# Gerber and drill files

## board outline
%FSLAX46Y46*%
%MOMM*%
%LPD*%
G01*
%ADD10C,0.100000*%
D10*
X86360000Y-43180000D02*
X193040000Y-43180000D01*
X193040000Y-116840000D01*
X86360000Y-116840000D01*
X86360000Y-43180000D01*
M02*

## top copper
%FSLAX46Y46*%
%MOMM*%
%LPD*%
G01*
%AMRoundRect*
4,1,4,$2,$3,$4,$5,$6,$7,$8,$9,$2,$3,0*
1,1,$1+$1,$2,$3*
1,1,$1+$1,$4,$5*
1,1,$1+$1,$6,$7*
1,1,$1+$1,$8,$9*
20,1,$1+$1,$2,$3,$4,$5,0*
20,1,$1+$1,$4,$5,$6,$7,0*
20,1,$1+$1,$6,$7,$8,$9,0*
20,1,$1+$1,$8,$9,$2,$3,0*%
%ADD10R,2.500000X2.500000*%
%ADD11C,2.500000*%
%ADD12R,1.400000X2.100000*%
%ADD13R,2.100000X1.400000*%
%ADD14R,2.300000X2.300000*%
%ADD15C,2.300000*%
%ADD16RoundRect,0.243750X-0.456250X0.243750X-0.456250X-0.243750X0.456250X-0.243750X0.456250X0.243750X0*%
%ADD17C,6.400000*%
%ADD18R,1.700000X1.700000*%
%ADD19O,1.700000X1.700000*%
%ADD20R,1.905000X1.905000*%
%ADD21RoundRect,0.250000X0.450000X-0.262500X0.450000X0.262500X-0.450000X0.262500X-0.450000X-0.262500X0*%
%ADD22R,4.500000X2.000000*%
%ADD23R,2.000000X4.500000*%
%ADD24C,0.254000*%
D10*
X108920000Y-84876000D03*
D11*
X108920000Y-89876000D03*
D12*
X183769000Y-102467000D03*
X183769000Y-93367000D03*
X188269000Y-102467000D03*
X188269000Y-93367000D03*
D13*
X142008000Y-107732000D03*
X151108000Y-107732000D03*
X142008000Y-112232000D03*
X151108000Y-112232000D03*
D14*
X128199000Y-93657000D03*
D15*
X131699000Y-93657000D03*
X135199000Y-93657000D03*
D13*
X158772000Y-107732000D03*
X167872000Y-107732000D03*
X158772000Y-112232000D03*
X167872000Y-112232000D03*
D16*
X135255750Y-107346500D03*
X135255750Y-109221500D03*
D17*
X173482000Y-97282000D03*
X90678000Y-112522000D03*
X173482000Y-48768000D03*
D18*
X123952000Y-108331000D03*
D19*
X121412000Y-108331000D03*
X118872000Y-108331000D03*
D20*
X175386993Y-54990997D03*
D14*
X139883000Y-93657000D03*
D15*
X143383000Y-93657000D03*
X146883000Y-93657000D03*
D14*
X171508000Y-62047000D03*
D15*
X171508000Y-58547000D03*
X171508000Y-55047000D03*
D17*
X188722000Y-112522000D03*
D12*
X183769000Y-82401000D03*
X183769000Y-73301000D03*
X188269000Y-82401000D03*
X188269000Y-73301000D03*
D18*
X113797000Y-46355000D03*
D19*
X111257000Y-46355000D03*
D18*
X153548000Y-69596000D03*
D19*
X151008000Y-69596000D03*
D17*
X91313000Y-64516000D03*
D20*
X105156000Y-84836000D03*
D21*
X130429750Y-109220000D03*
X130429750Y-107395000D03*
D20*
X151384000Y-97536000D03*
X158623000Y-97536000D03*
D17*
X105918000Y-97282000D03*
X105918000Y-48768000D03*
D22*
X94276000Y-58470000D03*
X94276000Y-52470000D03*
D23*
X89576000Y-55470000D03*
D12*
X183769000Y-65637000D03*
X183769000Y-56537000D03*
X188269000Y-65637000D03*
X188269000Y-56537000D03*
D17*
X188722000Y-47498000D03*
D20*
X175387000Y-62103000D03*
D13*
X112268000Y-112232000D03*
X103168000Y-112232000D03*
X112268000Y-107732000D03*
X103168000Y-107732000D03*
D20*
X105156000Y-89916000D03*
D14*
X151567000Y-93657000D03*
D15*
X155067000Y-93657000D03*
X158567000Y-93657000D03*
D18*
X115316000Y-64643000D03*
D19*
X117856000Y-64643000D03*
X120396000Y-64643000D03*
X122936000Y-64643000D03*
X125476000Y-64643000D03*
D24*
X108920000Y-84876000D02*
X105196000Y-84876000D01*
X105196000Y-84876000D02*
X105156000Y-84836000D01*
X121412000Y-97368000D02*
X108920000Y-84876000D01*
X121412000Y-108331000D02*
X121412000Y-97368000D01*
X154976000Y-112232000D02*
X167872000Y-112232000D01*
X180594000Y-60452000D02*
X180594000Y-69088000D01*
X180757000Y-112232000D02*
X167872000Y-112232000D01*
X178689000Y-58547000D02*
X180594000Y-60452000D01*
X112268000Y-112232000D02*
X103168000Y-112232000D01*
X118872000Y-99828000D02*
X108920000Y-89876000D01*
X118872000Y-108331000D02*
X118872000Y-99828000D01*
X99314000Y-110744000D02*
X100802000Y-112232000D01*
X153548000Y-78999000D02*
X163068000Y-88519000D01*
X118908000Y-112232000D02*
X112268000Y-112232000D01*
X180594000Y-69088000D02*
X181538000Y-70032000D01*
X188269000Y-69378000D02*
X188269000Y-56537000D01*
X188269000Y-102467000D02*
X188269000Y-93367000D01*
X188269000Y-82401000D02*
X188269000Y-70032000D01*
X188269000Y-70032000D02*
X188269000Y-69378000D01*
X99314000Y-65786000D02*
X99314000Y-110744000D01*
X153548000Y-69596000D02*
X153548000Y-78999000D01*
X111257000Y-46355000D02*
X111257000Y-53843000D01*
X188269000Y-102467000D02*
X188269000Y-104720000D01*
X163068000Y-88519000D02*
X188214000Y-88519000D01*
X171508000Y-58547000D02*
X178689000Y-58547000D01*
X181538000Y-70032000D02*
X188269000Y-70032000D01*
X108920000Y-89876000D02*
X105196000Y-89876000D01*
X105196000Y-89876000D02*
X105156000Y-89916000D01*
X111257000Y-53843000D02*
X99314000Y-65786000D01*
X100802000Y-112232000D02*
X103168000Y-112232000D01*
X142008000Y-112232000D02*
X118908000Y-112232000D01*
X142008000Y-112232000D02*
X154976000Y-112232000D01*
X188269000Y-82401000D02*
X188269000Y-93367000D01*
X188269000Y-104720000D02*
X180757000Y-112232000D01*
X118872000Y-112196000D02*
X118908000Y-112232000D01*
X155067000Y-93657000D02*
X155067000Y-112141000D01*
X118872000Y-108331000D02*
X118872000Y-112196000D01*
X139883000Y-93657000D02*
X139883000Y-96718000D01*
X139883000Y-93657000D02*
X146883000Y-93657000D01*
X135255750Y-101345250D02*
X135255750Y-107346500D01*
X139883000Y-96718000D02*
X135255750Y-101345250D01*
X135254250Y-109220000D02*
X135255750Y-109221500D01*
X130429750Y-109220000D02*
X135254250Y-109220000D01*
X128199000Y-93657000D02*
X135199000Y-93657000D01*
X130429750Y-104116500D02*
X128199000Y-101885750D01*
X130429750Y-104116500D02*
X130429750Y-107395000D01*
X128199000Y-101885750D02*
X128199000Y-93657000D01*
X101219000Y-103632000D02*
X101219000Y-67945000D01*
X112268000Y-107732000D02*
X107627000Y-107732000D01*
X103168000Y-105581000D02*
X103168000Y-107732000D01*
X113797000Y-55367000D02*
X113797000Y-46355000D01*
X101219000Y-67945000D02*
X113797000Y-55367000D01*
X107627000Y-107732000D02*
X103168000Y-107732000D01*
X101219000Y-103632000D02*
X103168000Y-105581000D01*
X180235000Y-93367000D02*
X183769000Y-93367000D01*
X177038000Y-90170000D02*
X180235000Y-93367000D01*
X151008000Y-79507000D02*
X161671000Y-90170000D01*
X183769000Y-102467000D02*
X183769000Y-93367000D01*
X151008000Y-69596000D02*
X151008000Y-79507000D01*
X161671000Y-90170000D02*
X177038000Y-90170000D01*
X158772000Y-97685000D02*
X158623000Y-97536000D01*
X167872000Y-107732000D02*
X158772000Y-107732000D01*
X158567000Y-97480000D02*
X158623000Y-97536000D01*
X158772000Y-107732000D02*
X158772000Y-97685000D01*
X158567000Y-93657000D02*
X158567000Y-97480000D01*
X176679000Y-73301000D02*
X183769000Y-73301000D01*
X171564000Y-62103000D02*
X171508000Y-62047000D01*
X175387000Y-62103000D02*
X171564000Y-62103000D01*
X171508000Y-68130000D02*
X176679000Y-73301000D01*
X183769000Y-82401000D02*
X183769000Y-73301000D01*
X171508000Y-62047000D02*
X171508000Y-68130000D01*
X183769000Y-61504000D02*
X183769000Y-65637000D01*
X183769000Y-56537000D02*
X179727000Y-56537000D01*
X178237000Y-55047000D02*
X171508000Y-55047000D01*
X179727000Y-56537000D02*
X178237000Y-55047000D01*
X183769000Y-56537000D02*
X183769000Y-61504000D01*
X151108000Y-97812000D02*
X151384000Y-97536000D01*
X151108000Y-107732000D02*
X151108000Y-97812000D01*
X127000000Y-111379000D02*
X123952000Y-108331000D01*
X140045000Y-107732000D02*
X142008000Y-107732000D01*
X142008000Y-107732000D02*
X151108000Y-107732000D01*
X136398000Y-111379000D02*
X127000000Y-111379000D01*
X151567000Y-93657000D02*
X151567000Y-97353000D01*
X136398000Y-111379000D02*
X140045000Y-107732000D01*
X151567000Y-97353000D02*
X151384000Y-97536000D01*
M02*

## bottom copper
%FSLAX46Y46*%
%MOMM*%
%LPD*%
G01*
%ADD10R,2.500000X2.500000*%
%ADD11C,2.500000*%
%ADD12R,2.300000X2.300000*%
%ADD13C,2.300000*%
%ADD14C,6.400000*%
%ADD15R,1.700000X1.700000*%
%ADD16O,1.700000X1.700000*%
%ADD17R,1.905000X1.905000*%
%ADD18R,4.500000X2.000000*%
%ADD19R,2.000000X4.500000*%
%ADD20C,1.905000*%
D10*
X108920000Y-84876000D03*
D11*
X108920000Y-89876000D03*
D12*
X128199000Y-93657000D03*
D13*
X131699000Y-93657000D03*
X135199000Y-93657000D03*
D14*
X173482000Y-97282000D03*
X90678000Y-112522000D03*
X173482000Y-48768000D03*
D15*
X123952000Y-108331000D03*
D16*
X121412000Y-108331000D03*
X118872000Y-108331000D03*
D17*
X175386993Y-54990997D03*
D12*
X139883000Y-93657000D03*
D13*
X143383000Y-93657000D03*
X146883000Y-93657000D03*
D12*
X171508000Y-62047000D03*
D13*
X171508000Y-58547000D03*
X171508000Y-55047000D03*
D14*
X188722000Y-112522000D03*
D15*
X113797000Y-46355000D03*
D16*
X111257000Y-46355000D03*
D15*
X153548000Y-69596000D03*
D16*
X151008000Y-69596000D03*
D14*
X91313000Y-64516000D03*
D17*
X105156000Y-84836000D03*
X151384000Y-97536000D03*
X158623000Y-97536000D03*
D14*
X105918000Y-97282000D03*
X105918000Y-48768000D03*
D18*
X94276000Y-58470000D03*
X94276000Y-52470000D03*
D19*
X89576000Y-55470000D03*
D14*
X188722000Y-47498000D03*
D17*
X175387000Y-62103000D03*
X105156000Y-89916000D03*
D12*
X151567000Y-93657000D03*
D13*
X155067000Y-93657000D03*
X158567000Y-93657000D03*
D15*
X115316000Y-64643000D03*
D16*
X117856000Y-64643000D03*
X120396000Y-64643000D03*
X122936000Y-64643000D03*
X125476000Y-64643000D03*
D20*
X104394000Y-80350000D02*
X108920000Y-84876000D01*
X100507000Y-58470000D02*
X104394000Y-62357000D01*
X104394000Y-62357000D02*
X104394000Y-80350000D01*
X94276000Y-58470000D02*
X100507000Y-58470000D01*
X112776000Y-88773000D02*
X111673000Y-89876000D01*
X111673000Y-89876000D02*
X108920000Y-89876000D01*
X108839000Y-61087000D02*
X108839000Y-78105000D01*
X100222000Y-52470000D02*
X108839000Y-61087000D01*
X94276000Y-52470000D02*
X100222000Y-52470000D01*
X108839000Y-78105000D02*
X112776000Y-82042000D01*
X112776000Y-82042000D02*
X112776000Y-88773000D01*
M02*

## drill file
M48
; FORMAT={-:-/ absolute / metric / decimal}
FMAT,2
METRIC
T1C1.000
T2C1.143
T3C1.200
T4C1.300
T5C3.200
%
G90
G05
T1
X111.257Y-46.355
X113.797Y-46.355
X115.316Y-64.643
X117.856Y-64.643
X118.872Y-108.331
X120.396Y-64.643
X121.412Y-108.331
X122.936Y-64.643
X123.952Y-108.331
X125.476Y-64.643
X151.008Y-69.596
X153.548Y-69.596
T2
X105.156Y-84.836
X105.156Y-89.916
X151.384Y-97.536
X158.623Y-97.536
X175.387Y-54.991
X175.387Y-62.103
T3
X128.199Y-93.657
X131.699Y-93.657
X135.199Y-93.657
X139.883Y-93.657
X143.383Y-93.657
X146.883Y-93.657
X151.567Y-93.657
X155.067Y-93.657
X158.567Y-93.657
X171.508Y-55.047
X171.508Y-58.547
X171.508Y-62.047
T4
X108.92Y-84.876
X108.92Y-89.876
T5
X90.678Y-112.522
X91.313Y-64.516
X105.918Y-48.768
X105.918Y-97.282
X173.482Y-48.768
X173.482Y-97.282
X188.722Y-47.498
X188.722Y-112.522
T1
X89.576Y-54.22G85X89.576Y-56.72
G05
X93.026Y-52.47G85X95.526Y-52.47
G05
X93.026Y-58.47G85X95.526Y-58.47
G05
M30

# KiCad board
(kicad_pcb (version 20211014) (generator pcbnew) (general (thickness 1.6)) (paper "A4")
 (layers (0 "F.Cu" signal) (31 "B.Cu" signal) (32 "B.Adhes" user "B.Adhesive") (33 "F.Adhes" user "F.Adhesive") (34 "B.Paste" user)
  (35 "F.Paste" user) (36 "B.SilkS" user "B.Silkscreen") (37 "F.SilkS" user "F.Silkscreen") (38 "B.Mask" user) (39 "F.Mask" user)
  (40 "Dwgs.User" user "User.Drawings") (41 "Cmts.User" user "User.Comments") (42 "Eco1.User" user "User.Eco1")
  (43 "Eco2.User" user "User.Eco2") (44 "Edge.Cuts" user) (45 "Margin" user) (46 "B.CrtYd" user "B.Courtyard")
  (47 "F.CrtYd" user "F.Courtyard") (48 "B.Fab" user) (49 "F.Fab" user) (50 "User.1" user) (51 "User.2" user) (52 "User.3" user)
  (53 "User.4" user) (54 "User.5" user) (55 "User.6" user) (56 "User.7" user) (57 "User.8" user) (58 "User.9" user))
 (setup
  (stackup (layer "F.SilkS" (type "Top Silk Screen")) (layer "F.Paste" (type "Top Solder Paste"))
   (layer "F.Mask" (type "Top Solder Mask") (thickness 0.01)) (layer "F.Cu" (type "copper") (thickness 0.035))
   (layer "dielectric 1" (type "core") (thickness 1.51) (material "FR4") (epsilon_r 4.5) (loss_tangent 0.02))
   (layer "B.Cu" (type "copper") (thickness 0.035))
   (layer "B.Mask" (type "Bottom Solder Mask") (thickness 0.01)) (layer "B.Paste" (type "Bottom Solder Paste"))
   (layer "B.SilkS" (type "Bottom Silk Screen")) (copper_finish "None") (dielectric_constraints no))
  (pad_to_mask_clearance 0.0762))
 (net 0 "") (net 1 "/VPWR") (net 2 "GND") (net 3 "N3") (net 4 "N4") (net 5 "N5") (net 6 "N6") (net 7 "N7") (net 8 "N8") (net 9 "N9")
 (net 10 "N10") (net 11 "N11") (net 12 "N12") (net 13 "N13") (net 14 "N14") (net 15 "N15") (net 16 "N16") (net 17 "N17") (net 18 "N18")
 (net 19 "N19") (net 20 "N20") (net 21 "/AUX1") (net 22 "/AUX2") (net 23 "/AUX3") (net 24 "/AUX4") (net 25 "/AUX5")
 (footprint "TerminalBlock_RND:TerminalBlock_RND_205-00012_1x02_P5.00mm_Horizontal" (layer "F.Cu") (at 108.92 84.876 -90)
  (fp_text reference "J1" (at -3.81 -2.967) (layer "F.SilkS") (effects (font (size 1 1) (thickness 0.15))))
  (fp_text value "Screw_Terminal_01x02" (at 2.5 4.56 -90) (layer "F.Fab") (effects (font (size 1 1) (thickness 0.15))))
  (pad "1" thru_hole rect (at 0 0 270) (size 2.5 2.5) (drill 1.3) (layers *.Cu *.Mask) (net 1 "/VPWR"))
  (pad "2" thru_hole circle (at 5 0 270) (size 2.5 2.5) (drill 1.3) (layers *.Cu *.Mask) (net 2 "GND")))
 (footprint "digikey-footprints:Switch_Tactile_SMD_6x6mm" (layer "F.Cu") (at 186.019 97.917 90)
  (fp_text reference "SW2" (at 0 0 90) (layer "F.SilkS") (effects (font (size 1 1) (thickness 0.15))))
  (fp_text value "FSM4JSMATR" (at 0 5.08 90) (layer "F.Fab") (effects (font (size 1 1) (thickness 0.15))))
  (pad "1" smd rect locked (at -4.55 -2.25) (size 1.4 2.1) (layers "F.Cu" "F.Paste" "F.Mask") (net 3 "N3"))
  (pad "2" smd rect locked (at 4.55 -2.25) (size 1.4 2.1) (layers "F.Cu" "F.Paste" "F.Mask") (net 3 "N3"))
  (pad "3" smd rect locked (at -4.55 2.25) (size 1.4 2.1) (layers "F.Cu" "F.Paste" "F.Mask") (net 2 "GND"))
  (pad "4" smd rect locked (at 4.55 2.25) (size 1.4 2.1) (layers "F.Cu" "F.Paste" "F.Mask") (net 2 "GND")))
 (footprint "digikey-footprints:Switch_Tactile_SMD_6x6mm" (layer "F.Cu") (at 146.558 109.982)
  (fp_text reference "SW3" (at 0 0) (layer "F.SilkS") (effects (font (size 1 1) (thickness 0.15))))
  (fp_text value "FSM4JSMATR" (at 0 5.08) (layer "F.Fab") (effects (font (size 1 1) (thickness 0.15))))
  (pad "1" smd rect locked (at -4.55 -2.25 270) (size 1.4 2.1) (layers "F.Cu" "F.Paste" "F.Mask") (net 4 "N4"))
  (pad "2" smd rect locked (at 4.55 -2.25 270) (size 1.4 2.1) (layers "F.Cu" "F.Paste" "F.Mask") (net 4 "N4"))
  (pad "3" smd rect locked (at -4.55 2.25 270) (size 1.4 2.1) (layers "F.Cu" "F.Paste" "F.Mask") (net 2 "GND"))
  (pad "4" smd rect locked (at 4.55 2.25 270) (size 1.4 2.1) (layers "F.Cu" "F.Paste" "F.Mask") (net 2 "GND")))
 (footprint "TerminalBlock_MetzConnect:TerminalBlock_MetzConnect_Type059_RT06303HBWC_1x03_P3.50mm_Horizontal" (layer "F.Cu")
  (at 128.199 93.657)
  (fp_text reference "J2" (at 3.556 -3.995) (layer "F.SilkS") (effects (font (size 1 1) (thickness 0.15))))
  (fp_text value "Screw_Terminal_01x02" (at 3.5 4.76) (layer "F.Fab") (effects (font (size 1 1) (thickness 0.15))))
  (pad "1" thru_hole rect (at 0 0) (size 2.3 2.3) (drill 1.2) (layers *.Cu *.Mask) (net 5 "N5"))
  (pad "2" thru_hole circle (at 3.5 0) (size 2.3 2.3) (drill 1.2) (layers *.Cu *.Mask) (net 5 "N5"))
  (pad "3" thru_hole circle (at 7 0) (size 2.3 2.3) (drill 1.2) (layers *.Cu *.Mask) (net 5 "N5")))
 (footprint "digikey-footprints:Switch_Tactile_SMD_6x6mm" (layer "F.Cu") (at 163.322 109.982)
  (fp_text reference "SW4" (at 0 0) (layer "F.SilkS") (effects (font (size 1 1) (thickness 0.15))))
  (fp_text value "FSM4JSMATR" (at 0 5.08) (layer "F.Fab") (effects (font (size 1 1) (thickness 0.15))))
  (pad "1" smd rect locked (at -4.55 -2.25 270) (size 1.4 2.1) (layers "F.Cu" "F.Paste" "F.Mask") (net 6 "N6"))
  (pad "2" smd rect locked (at 4.55 -2.25 270) (size 1.4 2.1) (layers "F.Cu" "F.Paste" "F.Mask") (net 6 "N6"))
  (pad "3" smd rect locked (at -4.55 2.25 270) (size 1.4 2.1) (layers "F.Cu" "F.Paste" "F.Mask") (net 2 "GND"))
  (pad "4" smd rect locked (at 4.55 2.25 270) (size 1.4 2.1) (layers "F.Cu" "F.Paste" "F.Mask") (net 2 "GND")))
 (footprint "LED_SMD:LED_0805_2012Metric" (layer "F.Cu") (at 135.25575 108.284 -90)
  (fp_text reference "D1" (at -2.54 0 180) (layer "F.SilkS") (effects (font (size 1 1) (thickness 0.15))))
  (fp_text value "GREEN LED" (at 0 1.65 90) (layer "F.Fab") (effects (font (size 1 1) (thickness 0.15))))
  (pad "1" smd roundrect (at -0.9375 0 270) (size 0.975 1.4) (layers "F.Cu" "F.Paste" "F.Mask") (roundrect_rratio 0.25) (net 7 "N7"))
  (pad "2" smd roundrect (at 0.9375 0 270) (size 0.975 1.4) (layers "F.Cu" "F.Paste" "F.Mask") (roundrect_rratio 0.25) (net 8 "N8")))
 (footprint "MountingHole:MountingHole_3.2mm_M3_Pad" (layer "F.Cu") (at 173.482 97.282)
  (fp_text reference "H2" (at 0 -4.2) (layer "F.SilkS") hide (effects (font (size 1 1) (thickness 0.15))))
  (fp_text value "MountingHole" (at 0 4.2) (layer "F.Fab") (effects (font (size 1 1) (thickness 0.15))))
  (pad "1" thru_hole circle (at 0 0) (size 6.4 6.4) (drill 3.2) (layers *.Cu *.Mask) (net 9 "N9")))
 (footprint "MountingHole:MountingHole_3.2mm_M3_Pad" (layer "F.Cu") (at 90.678 112.522)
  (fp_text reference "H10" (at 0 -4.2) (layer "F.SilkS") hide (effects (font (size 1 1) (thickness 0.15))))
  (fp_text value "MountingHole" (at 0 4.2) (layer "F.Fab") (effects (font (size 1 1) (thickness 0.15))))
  (pad "1" thru_hole circle (at 0 0) (size 6.4 6.4) (drill 3.2) (layers *.Cu *.Mask) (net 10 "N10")))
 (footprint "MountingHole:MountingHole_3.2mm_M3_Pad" (layer "F.Cu") (at 173.482 48.768)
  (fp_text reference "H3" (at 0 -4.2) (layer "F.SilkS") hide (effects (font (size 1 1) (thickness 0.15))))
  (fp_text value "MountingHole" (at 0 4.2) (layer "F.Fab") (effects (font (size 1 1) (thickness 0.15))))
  (pad "1" thru_hole circle (at 0 0) (size 6.4 6.4) (drill 3.2) (layers *.Cu *.Mask) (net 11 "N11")))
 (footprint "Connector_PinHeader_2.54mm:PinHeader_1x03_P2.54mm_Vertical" (layer "F.Cu") (at 123.952 108.331 -90)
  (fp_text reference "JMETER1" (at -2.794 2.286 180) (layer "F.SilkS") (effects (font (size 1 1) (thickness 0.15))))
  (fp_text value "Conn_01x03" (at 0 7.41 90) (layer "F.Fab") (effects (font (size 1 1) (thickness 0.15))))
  (pad "1" thru_hole rect (at 0 0 270) (size 1.7 1.7) (drill 1) (layers *.Cu *.Mask) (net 4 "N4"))
  (pad "2" thru_hole oval (at 0 2.54 270) (size 1.7 1.7) (drill 1) (layers *.Cu *.Mask) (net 1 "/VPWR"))
  (pad "3" thru_hole oval (at 0 5.08 270) (size 1.7 1.7) (drill 1) (layers *.Cu *.Mask) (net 2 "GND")))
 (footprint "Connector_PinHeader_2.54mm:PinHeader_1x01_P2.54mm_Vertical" (layer "F.Cu") (at 175.387 54.991)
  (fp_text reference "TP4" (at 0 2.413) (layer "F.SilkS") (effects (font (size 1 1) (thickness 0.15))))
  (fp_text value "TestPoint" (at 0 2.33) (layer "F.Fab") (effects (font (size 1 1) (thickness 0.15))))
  (pad "1" thru_hole rect (at -0.000007 -0.000003) (size 1.905 1.905) (drill 1.143) (layers *.Cu *.Mask) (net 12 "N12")))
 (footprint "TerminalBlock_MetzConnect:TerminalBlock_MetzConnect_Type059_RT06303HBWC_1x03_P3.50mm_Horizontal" (layer "F.Cu")
  (at 139.883 93.657)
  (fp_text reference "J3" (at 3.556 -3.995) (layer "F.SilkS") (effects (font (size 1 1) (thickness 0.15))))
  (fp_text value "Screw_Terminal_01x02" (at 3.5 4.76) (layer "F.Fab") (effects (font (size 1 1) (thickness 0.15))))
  (pad "1" thru_hole rect (at 0 0) (size 2.3 2.3) (drill 1.2) (layers *.Cu *.Mask) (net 7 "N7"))
  (pad "2" thru_hole circle (at 3.5 0) (size 2.3 2.3) (drill 1.2) (layers *.Cu *.Mask) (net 7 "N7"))
  (pad "3" thru_hole circle (at 7 0) (size 2.3 2.3) (drill 1.2) (layers *.Cu *.Mask) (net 7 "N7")))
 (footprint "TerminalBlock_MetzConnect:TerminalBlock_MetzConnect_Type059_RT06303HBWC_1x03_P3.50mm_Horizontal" (layer "F.Cu")
  (at 171.508 62.047 90)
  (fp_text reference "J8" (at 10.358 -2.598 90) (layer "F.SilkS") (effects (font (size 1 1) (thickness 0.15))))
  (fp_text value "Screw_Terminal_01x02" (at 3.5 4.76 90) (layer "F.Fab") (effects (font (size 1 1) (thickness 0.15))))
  (pad "1" thru_hole rect (at 0 0 90) (size 2.3 2.3) (drill 1.2) (layers *.Cu *.Mask) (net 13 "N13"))
  (pad "2" thru_hole circle (at 3.5 0 90) (size 2.3 2.3) (drill 1.2) (layers *.Cu *.Mask) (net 2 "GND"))
  (pad "3" thru_hole circle (at 7 0 90) (size 2.3 2.3) (drill 1.2) (layers *.Cu *.Mask) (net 12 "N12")))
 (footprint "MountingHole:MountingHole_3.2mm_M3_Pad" (layer "F.Cu") (at 188.722 112.522)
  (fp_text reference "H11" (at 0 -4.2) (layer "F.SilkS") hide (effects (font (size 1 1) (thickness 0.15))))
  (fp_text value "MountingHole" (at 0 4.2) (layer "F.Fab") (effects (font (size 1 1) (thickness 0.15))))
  (pad "1" thru_hole circle (at 0 0) (size 6.4 6.4) (drill 3.2) (layers *.Cu *.Mask) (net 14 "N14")))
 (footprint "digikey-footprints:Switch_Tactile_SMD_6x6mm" (layer "F.Cu") (at 186.019 77.851 90)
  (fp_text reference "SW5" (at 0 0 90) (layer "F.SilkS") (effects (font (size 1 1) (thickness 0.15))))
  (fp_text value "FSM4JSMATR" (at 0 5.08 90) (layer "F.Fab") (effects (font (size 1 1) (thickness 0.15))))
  (pad "1" smd rect locked (at -4.55 -2.25) (size 1.4 2.1) (layers "F.Cu" "F.Paste" "F.Mask") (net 13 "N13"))
  (pad "2" smd rect locked (at 4.55 -2.25) (size 1.4 2.1) (layers "F.Cu" "F.Paste" "F.Mask") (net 13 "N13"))
  (pad "3" smd rect locked (at -4.55 2.25) (size 1.4 2.1) (layers "F.Cu" "F.Paste" "F.Mask") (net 2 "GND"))
  (pad "4" smd rect locked (at 4.55 2.25) (size 1.4 2.1) (layers "F.Cu" "F.Paste" "F.Mask") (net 2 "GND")))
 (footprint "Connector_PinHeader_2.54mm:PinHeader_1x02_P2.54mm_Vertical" (layer "F.Cu") (at 113.797 46.355 -90)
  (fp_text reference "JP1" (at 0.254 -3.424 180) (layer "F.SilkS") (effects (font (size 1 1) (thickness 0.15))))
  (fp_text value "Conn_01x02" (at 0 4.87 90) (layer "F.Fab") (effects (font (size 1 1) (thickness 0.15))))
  (pad "1" thru_hole rect (at 0 0 270) (size 1.7 1.7) (drill 1) (layers *.Cu *.Mask) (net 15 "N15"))
  (pad "2" thru_hole oval (at 0 2.54 270) (size 1.7 1.7) (drill 1) (layers *.Cu *.Mask) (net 2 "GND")))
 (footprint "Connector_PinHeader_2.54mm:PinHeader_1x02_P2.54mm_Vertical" (layer "F.Cu") (at 153.548 69.596 -90)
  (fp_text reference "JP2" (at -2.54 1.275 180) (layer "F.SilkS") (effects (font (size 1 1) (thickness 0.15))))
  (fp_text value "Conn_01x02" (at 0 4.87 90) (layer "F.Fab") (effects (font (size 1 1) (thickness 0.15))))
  (pad "1" thru_hole rect (at 0 0 270) (size 1.7 1.7) (drill 1) (layers *.Cu *.Mask) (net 2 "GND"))
  (pad "2" thru_hole oval (at 0 2.54 270) (size 1.7 1.7) (drill 1) (layers *.Cu *.Mask) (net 3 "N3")))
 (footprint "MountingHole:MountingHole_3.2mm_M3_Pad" (layer "F.Cu") (at 91.313 64.516)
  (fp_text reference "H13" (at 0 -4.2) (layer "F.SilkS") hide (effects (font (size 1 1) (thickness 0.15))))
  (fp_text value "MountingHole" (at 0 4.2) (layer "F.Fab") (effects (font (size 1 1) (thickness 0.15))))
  (pad "1" thru_hole circle (at 0 0) (size 6.4 6.4) (drill 3.2) (layers *.Cu *.Mask) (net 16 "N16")))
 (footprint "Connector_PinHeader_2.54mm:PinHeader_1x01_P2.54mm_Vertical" (layer "F.Cu") (at 105.156 84.836)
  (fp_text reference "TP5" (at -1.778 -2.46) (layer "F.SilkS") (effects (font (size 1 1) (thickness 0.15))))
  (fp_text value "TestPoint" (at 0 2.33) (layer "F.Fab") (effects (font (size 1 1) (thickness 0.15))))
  (pad "1" thru_hole rect (at 0 0) (size 1.905 1.905) (drill 1.143) (layers *.Cu *.Mask) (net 1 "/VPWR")))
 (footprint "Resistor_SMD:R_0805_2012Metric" (layer "F.Cu") (at 130.42975 108.3075 90)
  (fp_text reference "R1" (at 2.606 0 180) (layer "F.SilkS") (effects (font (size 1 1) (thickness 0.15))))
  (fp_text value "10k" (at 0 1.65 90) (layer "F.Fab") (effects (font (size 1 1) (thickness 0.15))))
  (pad "1" smd roundrect (at -0.9125 0 90) (size 1.025 1.4) (layers "F.Cu" "F.Paste" "F.Mask") (roundrect_rratio 0.243902) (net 8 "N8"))
  (pad "2" smd roundrect (at 0.9125 0 90) (size 1.025 1.4) (layers "F.Cu" "F.Paste" "F.Mask") (roundrect_rratio 0.243902) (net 5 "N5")))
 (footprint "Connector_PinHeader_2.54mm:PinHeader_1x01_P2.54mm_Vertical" (layer "F.Cu") (at 151.384 97.536)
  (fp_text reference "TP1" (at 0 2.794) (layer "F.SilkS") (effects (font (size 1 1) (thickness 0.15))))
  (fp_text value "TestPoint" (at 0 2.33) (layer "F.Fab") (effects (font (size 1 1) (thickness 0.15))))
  (pad "1" thru_hole rect (at 0 0) (size 1.905 1.905) (drill 1.143) (layers *.Cu *.Mask) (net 4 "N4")))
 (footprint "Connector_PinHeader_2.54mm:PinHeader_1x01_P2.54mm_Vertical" (layer "F.Cu") (at 158.623 97.536)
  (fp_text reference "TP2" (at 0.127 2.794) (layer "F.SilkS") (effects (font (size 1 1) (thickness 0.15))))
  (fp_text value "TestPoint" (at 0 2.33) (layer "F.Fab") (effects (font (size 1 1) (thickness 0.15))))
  (pad "1" thru_hole rect (at 0 0) (size 1.905 1.905) (drill 1.143) (layers *.Cu *.Mask) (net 6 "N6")))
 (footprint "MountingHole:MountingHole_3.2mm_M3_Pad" (layer "F.Cu") (at 105.918 97.282)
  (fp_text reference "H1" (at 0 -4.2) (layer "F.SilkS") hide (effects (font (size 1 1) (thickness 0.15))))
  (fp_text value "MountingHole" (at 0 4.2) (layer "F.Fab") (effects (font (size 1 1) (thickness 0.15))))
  (pad "1" thru_hole circle (at 0 0) (size 6.4 6.4) (drill 3.2) (layers *.Cu *.Mask) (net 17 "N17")))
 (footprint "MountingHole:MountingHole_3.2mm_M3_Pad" (layer "F.Cu") (at 105.918 48.768)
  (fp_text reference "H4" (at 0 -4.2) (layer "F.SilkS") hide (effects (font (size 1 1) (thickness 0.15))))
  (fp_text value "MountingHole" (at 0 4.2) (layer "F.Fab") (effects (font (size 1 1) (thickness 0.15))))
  (pad "1" thru_hole circle (at 0 0) (size 6.4 6.4) (drill 3.2) (layers *.Cu *.Mask) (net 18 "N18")))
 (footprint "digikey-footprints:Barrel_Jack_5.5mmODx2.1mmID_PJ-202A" (layer "F.Cu") (at 94.276 55.47)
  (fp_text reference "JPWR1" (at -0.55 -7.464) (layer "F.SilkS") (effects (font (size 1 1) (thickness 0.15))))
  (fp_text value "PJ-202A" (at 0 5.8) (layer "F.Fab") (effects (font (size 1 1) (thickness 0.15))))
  (pad "1" thru_hole rect locked (at 0 3) (size 4.5 2) (drill oval 3.5 1) (layers *.Cu *.Mask) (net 1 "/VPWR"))
  (pad "2" thru_hole rect locked (at 0 -3) (size 4.5 2) (drill oval 3.5 1) (layers *.Cu *.Mask) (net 2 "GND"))
  (pad "3" thru_hole rect locked (at -4.7 0) (size 2 4.5) (drill oval 1 3.5) (layers *.Cu *.Mask) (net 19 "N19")))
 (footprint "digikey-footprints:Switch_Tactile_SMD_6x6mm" (layer "F.Cu") (at 186.019 61.087 90)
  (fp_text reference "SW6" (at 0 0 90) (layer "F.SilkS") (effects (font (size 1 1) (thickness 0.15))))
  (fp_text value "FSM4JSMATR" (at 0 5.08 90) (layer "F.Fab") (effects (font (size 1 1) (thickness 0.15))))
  (pad "1" smd rect locked (at -4.55 -2.25) (size 1.4 2.1) (layers "F.Cu" "F.Paste" "F.Mask") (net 12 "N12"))
  (pad "2" smd rect locked (at 4.55 -2.25) (size 1.4 2.1) (layers "F.Cu" "F.Paste" "F.Mask") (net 12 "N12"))
  (pad "3" smd rect locked (at -4.55 2.25) (size 1.4 2.1) (layers "F.Cu" "F.Paste" "F.Mask") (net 2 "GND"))
  (pad "4" smd rect locked (at 4.55 2.25) (size 1.4 2.1) (layers "F.Cu" "F.Paste" "F.Mask") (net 2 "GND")))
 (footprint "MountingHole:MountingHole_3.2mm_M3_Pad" (layer "F.Cu") (at 188.722 47.498)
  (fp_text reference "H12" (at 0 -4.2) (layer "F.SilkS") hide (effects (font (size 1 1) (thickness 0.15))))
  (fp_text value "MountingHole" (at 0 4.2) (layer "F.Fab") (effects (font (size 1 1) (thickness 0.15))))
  (pad "1" thru_hole circle (at 0 0) (size 6.4 6.4) (drill 3.2) (layers *.Cu *.Mask) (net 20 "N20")))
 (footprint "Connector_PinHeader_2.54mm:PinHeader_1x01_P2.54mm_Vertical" (layer "F.Cu") (at 175.387007 62.103)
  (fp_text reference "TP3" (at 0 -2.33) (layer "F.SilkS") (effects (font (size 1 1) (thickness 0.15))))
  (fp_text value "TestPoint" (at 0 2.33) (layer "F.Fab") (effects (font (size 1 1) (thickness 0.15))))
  (pad "1" thru_hole rect (at -0.000007 0) (size 1.905 1.905) (drill 1.143) (layers *.Cu *.Mask) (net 13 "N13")))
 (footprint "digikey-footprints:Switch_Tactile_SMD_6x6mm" (layer "F.Cu") (at 107.718 109.982 180)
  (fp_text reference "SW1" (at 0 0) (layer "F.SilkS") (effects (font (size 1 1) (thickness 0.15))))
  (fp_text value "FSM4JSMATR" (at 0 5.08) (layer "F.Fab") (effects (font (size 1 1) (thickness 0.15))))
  (pad "1" smd rect locked (at -4.55 -2.25 90) (size 1.4 2.1) (layers "F.Cu" "F.Paste" "F.Mask") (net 2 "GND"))
  (pad "2" smd rect locked (at 4.55 -2.25 90) (size 1.4 2.1) (layers "F.Cu" "F.Paste" "F.Mask") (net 2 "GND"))
  (pad "3" smd rect locked (at -4.55 2.25 90) (size 1.4 2.1) (layers "F.Cu" "F.Paste" "F.Mask") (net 15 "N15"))
  (pad "4" smd rect locked (at 4.55 2.25 90) (size 1.4 2.1) (layers "F.Cu" "F.Paste" "F.Mask") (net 15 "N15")))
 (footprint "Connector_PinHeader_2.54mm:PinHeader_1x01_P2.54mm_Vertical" (layer "F.Cu") (at 105.156003 89.916)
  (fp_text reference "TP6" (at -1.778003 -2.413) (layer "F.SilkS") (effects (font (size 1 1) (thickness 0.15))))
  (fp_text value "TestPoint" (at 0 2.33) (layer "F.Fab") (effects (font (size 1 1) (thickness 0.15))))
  (pad "1" thru_hole rect (at -0.000003 0) (size 1.905 1.905) (drill 1.143) (layers *.Cu *.Mask) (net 2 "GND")))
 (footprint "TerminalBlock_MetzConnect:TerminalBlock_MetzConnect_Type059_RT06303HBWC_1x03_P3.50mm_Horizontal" (layer "F.Cu")
  (at 151.567 93.657)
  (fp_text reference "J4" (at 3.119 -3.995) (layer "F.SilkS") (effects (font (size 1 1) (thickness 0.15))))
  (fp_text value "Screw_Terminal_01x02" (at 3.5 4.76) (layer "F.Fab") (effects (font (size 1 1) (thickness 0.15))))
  (pad "1" thru_hole rect (at 0 0) (size 2.3 2.3) (drill 1.2) (layers *.Cu *.Mask) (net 4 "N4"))
  (pad "2" thru_hole circle (at 3.5 0) (size 2.3 2.3) (drill 1.2) (layers *.Cu *.Mask) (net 2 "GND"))
  (pad "3" thru_hole circle (at 7 0) (size 2.3 2.3) (drill 1.2) (layers *.Cu *.Mask) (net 6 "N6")))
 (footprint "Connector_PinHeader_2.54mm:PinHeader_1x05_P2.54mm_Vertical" (layer "F.Cu") (at 115.316 64.643 90)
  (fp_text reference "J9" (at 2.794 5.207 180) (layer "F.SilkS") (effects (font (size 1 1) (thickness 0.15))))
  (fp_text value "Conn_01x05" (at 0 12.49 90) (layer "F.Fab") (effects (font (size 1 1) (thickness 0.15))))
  (pad "1" thru_hole rect (at 0 0 90) (size 1.7 1.7) (drill 1) (layers *.Cu *.Mask) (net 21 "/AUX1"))
  (pad "2" thru_hole oval (at 0 2.54 90) (size 1.7 1.7) (drill 1) (layers *.Cu *.Mask) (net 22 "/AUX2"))
  (pad "3" thru_hole oval (at 0 5.08 90) (size 1.7 1.7) (drill 1) (layers *.Cu *.Mask) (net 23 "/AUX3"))
  (pad "4" thru_hole oval (at 0 7.62 90) (size 1.7 1.7) (drill 1) (layers *.Cu *.Mask) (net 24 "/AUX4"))
  (pad "5" thru_hole oval (at 0 10.16 90) (size 1.7 1.7) (drill 1) (layers *.Cu *.Mask) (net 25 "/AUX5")))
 (gr_rect (start 86.36 43.18) (end 193.04 116.84) (layer "Edge.Cuts") (width 0.1) (fill none))
 (segment (start 108.92 84.876) (end 105.196 84.876) (width 0.254) (layer "F.Cu") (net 1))
 (segment (start 105.196 84.876) (end 105.156 84.836) (width 0.254) (layer "F.Cu") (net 1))
 (segment (start 121.412 97.368) (end 108.92 84.876) (width 0.254) (layer "F.Cu") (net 1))
 (segment (start 121.412 108.331) (end 121.412 97.368) (width 0.254) (layer "F.Cu") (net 1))
 (segment (start 104.394 80.35) (end 108.92 84.876) (width 1.905) (layer "B.Cu") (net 1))
 (segment (start 100.507 58.47) (end 104.394 62.357) (width 1.905) (layer "B.Cu") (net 1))
 (segment (start 104.394 62.357) (end 104.394 80.35) (width 1.905) (layer "B.Cu") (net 1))
 (segment (start 94.276 58.47) (end 100.507 58.47) (width 1.905) (layer "B.Cu") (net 1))
 (segment (start 154.976 112.232) (end 167.872 112.232) (width 0.254) (layer "F.Cu") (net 2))
 (segment (start 180.594 60.452) (end 180.594 69.088) (width 0.254) (layer "F.Cu") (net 2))
 (segment (start 180.757 112.232) (end 167.872 112.232) (width 0.254) (layer "F.Cu") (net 2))
 (segment (start 178.689 58.547) (end 180.594 60.452) (width 0.254) (layer "F.Cu") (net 2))
 (segment (start 112.268 112.232) (end 103.168 112.232) (width 0.254) (layer "F.Cu") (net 2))
 (segment (start 118.872 99.828) (end 108.92 89.876) (width 0.254) (layer "F.Cu") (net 2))
 (segment (start 118.872 108.331) (end 118.872 99.828) (width 0.254) (layer "F.Cu") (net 2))
 (segment (start 99.314 110.744) (end 100.802 112.232) (width 0.254) (layer "F.Cu") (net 2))
 (segment (start 153.548 78.999) (end 163.068 88.519) (width 0.254) (layer "F.Cu") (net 2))
 (segment (start 118.908 112.232) (end 112.268 112.232) (width 0.254) (layer "F.Cu") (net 2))
 (segment (start 180.594 69.088) (end 181.538 70.032) (width 0.254) (layer "F.Cu") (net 2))
 (segment (start 188.269 69.378) (end 188.269 56.537) (width 0.254) (layer "F.Cu") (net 2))
 (segment (start 188.269 102.467) (end 188.269 93.367) (width 0.254) (layer "F.Cu") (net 2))
 (segment (start 188.269 82.401) (end 188.269 70.032) (width 0.254) (layer "F.Cu") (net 2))
 (segment (start 188.269 70.032) (end 188.269 69.378) (width 0.254) (layer "F.Cu") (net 2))
 (segment (start 99.314 65.786) (end 99.314 110.744) (width 0.254) (layer "F.Cu") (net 2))
 (segment (start 153.548 69.596) (end 153.548 78.999) (width 0.254) (layer "F.Cu") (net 2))
 (segment (start 111.257 46.355) (end 111.257 53.843) (width 0.254) (layer "F.Cu") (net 2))
 (segment (start 188.269 102.467) (end 188.269 104.72) (width 0.254) (layer "F.Cu") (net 2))
 (segment (start 163.068 88.519) (end 188.214 88.519) (width 0.254) (layer "F.Cu") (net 2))
 (segment (start 171.508 58.547) (end 178.689 58.547) (width 0.254) (layer "F.Cu") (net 2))
 (segment (start 181.538 70.032) (end 188.269 70.032) (width 0.254) (layer "F.Cu") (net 2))
 (segment (start 108.92 89.876) (end 105.196 89.876) (width 0.254) (layer "F.Cu") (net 2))
 (segment (start 105.196 89.876) (end 105.156 89.916) (width 0.254) (layer "F.Cu") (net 2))
 (segment (start 111.257 53.843) (end 99.314 65.786) (width 0.254) (layer "F.Cu") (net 2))
 (segment (start 100.802 112.232) (end 103.168 112.232) (width 0.254) (layer "F.Cu") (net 2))
 (segment (start 142.008 112.232) (end 118.908 112.232) (width 0.254) (layer "F.Cu") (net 2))
 (segment (start 142.008 112.232) (end 154.976 112.232) (width 0.254) (layer "F.Cu") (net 2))
 (segment (start 188.269 82.401) (end 188.269 93.367) (width 0.254) (layer "F.Cu") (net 2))
 (segment (start 188.269 104.72) (end 180.757 112.232) (width 0.254) (layer "F.Cu") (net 2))
 (segment (start 118.872 112.196) (end 118.908 112.232) (width 0.254) (layer "F.Cu") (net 2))
 (segment (start 155.067 93.657) (end 155.067 112.141) (width 0.254) (layer "F.Cu") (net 2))
 (segment (start 118.872 108.331) (end 118.872 112.196) (width 0.254) (layer "F.Cu") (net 2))
 (segment (start 112.776 88.773) (end 111.673 89.876) (width 1.905) (layer "B.Cu") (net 2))
 (segment (start 111.673 89.876) (end 108.92 89.876) (width 1.905) (layer "B.Cu") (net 2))
 (segment (start 108.839 61.087) (end 108.839 78.105) (width 1.905) (layer "B.Cu") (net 2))
 (segment (start 100.222 52.47) (end 108.839 61.087) (width 1.905) (layer "B.Cu") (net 2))
 (segment (start 94.276 52.47) (end 100.222 52.47) (width 1.905) (layer "B.Cu") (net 2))
 (segment (start 108.839 78.105) (end 112.776 82.042) (width 1.905) (layer "B.Cu") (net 2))
 (segment (start 112.776 82.042) (end 112.776 88.773) (width 1.905) (layer "B.Cu") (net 2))
 (segment (start 139.883 93.657) (end 139.883 96.718) (width 0.254) (layer "F.Cu") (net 7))
 (segment (start 139.883 93.657) (end 146.883 93.657) (width 0.254) (layer "F.Cu") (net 7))
 (segment (start 135.25575 101.34525) (end 135.25575 107.3465) (width 0.254) (layer "F.Cu") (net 7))
 (segment (start 139.883 96.718) (end 135.25575 101.34525) (width 0.254) (layer "F.Cu") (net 7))
 (segment (start 135.25425 109.22) (end 135.25575 109.2215) (width 0.254) (layer "F.Cu") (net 8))
 (segment (start 130.42975 109.22) (end 135.25425 109.22) (width 0.254) (layer "F.Cu") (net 8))
 (segment (start 128.199 93.657) (end 135.199 93.657) (width 0.254) (layer "F.Cu") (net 5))
 (segment (start 130.42975 104.1165) (end 128.199 101.88575) (width 0.254) (layer "F.Cu") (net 5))
 (segment (start 130.42975 104.1165) (end 130.42975 107.395) (width 0.254) (layer "F.Cu") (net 5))
 (segment (start 128.199 101.88575) (end 128.199 93.657) (width 0.254) (layer "F.Cu") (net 5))
 (segment (start 101.219 103.632) (end 101.219 67.945) (width 0.254) (layer "F.Cu") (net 15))
 (segment (start 112.268 107.732) (end 107.627 107.732) (width 0.254) (layer "F.Cu") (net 15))
 (segment (start 103.168 105.581) (end 103.168 107.732) (width 0.254) (layer "F.Cu") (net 15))
 (segment (start 113.797 55.367) (end 113.797 46.355) (width 0.254) (layer "F.Cu") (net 15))
 (segment (start 101.219 67.945) (end 113.797 55.367) (width 0.254) (layer "F.Cu") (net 15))
 (segment (start 107.627 107.732) (end 103.168 107.732) (width 0.254) (layer "F.Cu") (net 15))
 (segment (start 101.219 103.632) (end 103.168 105.581) (width 0.254) (layer "F.Cu") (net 15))
 (segment (start 180.235 93.367) (end 183.769 93.367) (width 0.254) (layer "F.Cu") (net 3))
 (segment (start 177.038 90.17) (end 180.235 93.367) (width 0.254) (layer "F.Cu") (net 3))
 (segment (start 151.008 79.507) (end 161.671 90.17) (width 0.254) (layer "F.Cu") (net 3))
 (segment (start 183.769 102.467) (end 183.769 93.367) (width 0.254) (layer "F.Cu") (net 3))
 (segment (start 151.008 69.596) (end 151.008 79.507) (width 0.254) (layer "F.Cu") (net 3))
 (segment (start 161.671 90.17) (end 177.038 90.17) (width 0.254) (layer "F.Cu") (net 3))
 (segment (start 158.772 97.685) (end 158.623 97.536) (width 0.254) (layer "F.Cu") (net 6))
 (segment (start 167.872 107.732) (end 158.772 107.732) (width 0.254) (layer "F.Cu") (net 6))
 (segment (start 158.567 97.48) (end 158.623 97.536) (width 0.254) (layer "F.Cu") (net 6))
 (segment (start 158.772 107.732) (end 158.772 97.685) (width 0.254) (layer "F.Cu") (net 6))
 (segment (start 158.567 93.657) (end 158.567 97.48) (width 0.254) (layer "F.Cu") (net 6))
 (segment (start 176.679 73.301) (end 183.769 73.301) (width 0.254) (layer "F.Cu") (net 13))
 (segment (start 171.564 62.103) (end 171.508 62.047) (width 0.254) (layer "F.Cu") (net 13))
 (segment (start 175.387 62.103) (end 171.564 62.103) (width 0.254) (layer "F.Cu") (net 13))
 (segment (start 171.508 68.13) (end 176.679 73.301) (width 0.254) (layer "F.Cu") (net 13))
 (segment (start 183.769 82.401) (end 183.769 73.301) (width 0.254) (layer "F.Cu") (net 13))
 (segment (start 171.508 62.047) (end 171.508 68.13) (width 0.254) (layer "F.Cu") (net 13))
 (segment (start 183.769 61.504) (end 183.769 65.637) (width 0.254) (layer "F.Cu") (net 12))
 (segment (start 183.769 56.537) (end 179.727 56.537) (width 0.254) (layer "F.Cu") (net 12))
 (segment (start 178.237 55.047) (end 171.508 55.047) (width 0.254) (layer "F.Cu") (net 12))
 (segment (start 179.727 56.537) (end 178.237 55.047) (width 0.254) (layer "F.Cu") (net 12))
 (segment (start 183.769 56.537) (end 183.769 61.504) (width 0.254) (layer "F.Cu") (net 12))
 (segment (start 151.108 97.812) (end 151.384 97.536) (width 0.254) (layer "F.Cu") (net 4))
 (segment (start 151.108 107.732) (end 151.108 97.812) (width 0.254) (layer "F.Cu") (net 4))
 (segment (start 127 111.379) (end 123.952 108.331) (width 0.254) (layer "F.Cu") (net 4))
 (segment (start 140.045 107.732) (end 142.008 107.732) (width 0.254) (layer "F.Cu") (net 4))
 (segment (start 142.008 107.732) (end 151.108 107.732) (width 0.254) (layer "F.Cu") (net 4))
 (segment (start 136.398 111.379) (end 127 111.379) (width 0.254) (layer "F.Cu") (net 4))
 (segment (start 151.567 93.657) (end 151.567 97.353) (width 0.254) (layer "F.Cu") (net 4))
 (segment (start 136.398 111.379) (end 140.045 107.732) (width 0.254) (layer "F.Cu") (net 4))
 (segment (start 151.567 97.353) (end 151.384 97.536) (width 0.254) (layer "F.Cu") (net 4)))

